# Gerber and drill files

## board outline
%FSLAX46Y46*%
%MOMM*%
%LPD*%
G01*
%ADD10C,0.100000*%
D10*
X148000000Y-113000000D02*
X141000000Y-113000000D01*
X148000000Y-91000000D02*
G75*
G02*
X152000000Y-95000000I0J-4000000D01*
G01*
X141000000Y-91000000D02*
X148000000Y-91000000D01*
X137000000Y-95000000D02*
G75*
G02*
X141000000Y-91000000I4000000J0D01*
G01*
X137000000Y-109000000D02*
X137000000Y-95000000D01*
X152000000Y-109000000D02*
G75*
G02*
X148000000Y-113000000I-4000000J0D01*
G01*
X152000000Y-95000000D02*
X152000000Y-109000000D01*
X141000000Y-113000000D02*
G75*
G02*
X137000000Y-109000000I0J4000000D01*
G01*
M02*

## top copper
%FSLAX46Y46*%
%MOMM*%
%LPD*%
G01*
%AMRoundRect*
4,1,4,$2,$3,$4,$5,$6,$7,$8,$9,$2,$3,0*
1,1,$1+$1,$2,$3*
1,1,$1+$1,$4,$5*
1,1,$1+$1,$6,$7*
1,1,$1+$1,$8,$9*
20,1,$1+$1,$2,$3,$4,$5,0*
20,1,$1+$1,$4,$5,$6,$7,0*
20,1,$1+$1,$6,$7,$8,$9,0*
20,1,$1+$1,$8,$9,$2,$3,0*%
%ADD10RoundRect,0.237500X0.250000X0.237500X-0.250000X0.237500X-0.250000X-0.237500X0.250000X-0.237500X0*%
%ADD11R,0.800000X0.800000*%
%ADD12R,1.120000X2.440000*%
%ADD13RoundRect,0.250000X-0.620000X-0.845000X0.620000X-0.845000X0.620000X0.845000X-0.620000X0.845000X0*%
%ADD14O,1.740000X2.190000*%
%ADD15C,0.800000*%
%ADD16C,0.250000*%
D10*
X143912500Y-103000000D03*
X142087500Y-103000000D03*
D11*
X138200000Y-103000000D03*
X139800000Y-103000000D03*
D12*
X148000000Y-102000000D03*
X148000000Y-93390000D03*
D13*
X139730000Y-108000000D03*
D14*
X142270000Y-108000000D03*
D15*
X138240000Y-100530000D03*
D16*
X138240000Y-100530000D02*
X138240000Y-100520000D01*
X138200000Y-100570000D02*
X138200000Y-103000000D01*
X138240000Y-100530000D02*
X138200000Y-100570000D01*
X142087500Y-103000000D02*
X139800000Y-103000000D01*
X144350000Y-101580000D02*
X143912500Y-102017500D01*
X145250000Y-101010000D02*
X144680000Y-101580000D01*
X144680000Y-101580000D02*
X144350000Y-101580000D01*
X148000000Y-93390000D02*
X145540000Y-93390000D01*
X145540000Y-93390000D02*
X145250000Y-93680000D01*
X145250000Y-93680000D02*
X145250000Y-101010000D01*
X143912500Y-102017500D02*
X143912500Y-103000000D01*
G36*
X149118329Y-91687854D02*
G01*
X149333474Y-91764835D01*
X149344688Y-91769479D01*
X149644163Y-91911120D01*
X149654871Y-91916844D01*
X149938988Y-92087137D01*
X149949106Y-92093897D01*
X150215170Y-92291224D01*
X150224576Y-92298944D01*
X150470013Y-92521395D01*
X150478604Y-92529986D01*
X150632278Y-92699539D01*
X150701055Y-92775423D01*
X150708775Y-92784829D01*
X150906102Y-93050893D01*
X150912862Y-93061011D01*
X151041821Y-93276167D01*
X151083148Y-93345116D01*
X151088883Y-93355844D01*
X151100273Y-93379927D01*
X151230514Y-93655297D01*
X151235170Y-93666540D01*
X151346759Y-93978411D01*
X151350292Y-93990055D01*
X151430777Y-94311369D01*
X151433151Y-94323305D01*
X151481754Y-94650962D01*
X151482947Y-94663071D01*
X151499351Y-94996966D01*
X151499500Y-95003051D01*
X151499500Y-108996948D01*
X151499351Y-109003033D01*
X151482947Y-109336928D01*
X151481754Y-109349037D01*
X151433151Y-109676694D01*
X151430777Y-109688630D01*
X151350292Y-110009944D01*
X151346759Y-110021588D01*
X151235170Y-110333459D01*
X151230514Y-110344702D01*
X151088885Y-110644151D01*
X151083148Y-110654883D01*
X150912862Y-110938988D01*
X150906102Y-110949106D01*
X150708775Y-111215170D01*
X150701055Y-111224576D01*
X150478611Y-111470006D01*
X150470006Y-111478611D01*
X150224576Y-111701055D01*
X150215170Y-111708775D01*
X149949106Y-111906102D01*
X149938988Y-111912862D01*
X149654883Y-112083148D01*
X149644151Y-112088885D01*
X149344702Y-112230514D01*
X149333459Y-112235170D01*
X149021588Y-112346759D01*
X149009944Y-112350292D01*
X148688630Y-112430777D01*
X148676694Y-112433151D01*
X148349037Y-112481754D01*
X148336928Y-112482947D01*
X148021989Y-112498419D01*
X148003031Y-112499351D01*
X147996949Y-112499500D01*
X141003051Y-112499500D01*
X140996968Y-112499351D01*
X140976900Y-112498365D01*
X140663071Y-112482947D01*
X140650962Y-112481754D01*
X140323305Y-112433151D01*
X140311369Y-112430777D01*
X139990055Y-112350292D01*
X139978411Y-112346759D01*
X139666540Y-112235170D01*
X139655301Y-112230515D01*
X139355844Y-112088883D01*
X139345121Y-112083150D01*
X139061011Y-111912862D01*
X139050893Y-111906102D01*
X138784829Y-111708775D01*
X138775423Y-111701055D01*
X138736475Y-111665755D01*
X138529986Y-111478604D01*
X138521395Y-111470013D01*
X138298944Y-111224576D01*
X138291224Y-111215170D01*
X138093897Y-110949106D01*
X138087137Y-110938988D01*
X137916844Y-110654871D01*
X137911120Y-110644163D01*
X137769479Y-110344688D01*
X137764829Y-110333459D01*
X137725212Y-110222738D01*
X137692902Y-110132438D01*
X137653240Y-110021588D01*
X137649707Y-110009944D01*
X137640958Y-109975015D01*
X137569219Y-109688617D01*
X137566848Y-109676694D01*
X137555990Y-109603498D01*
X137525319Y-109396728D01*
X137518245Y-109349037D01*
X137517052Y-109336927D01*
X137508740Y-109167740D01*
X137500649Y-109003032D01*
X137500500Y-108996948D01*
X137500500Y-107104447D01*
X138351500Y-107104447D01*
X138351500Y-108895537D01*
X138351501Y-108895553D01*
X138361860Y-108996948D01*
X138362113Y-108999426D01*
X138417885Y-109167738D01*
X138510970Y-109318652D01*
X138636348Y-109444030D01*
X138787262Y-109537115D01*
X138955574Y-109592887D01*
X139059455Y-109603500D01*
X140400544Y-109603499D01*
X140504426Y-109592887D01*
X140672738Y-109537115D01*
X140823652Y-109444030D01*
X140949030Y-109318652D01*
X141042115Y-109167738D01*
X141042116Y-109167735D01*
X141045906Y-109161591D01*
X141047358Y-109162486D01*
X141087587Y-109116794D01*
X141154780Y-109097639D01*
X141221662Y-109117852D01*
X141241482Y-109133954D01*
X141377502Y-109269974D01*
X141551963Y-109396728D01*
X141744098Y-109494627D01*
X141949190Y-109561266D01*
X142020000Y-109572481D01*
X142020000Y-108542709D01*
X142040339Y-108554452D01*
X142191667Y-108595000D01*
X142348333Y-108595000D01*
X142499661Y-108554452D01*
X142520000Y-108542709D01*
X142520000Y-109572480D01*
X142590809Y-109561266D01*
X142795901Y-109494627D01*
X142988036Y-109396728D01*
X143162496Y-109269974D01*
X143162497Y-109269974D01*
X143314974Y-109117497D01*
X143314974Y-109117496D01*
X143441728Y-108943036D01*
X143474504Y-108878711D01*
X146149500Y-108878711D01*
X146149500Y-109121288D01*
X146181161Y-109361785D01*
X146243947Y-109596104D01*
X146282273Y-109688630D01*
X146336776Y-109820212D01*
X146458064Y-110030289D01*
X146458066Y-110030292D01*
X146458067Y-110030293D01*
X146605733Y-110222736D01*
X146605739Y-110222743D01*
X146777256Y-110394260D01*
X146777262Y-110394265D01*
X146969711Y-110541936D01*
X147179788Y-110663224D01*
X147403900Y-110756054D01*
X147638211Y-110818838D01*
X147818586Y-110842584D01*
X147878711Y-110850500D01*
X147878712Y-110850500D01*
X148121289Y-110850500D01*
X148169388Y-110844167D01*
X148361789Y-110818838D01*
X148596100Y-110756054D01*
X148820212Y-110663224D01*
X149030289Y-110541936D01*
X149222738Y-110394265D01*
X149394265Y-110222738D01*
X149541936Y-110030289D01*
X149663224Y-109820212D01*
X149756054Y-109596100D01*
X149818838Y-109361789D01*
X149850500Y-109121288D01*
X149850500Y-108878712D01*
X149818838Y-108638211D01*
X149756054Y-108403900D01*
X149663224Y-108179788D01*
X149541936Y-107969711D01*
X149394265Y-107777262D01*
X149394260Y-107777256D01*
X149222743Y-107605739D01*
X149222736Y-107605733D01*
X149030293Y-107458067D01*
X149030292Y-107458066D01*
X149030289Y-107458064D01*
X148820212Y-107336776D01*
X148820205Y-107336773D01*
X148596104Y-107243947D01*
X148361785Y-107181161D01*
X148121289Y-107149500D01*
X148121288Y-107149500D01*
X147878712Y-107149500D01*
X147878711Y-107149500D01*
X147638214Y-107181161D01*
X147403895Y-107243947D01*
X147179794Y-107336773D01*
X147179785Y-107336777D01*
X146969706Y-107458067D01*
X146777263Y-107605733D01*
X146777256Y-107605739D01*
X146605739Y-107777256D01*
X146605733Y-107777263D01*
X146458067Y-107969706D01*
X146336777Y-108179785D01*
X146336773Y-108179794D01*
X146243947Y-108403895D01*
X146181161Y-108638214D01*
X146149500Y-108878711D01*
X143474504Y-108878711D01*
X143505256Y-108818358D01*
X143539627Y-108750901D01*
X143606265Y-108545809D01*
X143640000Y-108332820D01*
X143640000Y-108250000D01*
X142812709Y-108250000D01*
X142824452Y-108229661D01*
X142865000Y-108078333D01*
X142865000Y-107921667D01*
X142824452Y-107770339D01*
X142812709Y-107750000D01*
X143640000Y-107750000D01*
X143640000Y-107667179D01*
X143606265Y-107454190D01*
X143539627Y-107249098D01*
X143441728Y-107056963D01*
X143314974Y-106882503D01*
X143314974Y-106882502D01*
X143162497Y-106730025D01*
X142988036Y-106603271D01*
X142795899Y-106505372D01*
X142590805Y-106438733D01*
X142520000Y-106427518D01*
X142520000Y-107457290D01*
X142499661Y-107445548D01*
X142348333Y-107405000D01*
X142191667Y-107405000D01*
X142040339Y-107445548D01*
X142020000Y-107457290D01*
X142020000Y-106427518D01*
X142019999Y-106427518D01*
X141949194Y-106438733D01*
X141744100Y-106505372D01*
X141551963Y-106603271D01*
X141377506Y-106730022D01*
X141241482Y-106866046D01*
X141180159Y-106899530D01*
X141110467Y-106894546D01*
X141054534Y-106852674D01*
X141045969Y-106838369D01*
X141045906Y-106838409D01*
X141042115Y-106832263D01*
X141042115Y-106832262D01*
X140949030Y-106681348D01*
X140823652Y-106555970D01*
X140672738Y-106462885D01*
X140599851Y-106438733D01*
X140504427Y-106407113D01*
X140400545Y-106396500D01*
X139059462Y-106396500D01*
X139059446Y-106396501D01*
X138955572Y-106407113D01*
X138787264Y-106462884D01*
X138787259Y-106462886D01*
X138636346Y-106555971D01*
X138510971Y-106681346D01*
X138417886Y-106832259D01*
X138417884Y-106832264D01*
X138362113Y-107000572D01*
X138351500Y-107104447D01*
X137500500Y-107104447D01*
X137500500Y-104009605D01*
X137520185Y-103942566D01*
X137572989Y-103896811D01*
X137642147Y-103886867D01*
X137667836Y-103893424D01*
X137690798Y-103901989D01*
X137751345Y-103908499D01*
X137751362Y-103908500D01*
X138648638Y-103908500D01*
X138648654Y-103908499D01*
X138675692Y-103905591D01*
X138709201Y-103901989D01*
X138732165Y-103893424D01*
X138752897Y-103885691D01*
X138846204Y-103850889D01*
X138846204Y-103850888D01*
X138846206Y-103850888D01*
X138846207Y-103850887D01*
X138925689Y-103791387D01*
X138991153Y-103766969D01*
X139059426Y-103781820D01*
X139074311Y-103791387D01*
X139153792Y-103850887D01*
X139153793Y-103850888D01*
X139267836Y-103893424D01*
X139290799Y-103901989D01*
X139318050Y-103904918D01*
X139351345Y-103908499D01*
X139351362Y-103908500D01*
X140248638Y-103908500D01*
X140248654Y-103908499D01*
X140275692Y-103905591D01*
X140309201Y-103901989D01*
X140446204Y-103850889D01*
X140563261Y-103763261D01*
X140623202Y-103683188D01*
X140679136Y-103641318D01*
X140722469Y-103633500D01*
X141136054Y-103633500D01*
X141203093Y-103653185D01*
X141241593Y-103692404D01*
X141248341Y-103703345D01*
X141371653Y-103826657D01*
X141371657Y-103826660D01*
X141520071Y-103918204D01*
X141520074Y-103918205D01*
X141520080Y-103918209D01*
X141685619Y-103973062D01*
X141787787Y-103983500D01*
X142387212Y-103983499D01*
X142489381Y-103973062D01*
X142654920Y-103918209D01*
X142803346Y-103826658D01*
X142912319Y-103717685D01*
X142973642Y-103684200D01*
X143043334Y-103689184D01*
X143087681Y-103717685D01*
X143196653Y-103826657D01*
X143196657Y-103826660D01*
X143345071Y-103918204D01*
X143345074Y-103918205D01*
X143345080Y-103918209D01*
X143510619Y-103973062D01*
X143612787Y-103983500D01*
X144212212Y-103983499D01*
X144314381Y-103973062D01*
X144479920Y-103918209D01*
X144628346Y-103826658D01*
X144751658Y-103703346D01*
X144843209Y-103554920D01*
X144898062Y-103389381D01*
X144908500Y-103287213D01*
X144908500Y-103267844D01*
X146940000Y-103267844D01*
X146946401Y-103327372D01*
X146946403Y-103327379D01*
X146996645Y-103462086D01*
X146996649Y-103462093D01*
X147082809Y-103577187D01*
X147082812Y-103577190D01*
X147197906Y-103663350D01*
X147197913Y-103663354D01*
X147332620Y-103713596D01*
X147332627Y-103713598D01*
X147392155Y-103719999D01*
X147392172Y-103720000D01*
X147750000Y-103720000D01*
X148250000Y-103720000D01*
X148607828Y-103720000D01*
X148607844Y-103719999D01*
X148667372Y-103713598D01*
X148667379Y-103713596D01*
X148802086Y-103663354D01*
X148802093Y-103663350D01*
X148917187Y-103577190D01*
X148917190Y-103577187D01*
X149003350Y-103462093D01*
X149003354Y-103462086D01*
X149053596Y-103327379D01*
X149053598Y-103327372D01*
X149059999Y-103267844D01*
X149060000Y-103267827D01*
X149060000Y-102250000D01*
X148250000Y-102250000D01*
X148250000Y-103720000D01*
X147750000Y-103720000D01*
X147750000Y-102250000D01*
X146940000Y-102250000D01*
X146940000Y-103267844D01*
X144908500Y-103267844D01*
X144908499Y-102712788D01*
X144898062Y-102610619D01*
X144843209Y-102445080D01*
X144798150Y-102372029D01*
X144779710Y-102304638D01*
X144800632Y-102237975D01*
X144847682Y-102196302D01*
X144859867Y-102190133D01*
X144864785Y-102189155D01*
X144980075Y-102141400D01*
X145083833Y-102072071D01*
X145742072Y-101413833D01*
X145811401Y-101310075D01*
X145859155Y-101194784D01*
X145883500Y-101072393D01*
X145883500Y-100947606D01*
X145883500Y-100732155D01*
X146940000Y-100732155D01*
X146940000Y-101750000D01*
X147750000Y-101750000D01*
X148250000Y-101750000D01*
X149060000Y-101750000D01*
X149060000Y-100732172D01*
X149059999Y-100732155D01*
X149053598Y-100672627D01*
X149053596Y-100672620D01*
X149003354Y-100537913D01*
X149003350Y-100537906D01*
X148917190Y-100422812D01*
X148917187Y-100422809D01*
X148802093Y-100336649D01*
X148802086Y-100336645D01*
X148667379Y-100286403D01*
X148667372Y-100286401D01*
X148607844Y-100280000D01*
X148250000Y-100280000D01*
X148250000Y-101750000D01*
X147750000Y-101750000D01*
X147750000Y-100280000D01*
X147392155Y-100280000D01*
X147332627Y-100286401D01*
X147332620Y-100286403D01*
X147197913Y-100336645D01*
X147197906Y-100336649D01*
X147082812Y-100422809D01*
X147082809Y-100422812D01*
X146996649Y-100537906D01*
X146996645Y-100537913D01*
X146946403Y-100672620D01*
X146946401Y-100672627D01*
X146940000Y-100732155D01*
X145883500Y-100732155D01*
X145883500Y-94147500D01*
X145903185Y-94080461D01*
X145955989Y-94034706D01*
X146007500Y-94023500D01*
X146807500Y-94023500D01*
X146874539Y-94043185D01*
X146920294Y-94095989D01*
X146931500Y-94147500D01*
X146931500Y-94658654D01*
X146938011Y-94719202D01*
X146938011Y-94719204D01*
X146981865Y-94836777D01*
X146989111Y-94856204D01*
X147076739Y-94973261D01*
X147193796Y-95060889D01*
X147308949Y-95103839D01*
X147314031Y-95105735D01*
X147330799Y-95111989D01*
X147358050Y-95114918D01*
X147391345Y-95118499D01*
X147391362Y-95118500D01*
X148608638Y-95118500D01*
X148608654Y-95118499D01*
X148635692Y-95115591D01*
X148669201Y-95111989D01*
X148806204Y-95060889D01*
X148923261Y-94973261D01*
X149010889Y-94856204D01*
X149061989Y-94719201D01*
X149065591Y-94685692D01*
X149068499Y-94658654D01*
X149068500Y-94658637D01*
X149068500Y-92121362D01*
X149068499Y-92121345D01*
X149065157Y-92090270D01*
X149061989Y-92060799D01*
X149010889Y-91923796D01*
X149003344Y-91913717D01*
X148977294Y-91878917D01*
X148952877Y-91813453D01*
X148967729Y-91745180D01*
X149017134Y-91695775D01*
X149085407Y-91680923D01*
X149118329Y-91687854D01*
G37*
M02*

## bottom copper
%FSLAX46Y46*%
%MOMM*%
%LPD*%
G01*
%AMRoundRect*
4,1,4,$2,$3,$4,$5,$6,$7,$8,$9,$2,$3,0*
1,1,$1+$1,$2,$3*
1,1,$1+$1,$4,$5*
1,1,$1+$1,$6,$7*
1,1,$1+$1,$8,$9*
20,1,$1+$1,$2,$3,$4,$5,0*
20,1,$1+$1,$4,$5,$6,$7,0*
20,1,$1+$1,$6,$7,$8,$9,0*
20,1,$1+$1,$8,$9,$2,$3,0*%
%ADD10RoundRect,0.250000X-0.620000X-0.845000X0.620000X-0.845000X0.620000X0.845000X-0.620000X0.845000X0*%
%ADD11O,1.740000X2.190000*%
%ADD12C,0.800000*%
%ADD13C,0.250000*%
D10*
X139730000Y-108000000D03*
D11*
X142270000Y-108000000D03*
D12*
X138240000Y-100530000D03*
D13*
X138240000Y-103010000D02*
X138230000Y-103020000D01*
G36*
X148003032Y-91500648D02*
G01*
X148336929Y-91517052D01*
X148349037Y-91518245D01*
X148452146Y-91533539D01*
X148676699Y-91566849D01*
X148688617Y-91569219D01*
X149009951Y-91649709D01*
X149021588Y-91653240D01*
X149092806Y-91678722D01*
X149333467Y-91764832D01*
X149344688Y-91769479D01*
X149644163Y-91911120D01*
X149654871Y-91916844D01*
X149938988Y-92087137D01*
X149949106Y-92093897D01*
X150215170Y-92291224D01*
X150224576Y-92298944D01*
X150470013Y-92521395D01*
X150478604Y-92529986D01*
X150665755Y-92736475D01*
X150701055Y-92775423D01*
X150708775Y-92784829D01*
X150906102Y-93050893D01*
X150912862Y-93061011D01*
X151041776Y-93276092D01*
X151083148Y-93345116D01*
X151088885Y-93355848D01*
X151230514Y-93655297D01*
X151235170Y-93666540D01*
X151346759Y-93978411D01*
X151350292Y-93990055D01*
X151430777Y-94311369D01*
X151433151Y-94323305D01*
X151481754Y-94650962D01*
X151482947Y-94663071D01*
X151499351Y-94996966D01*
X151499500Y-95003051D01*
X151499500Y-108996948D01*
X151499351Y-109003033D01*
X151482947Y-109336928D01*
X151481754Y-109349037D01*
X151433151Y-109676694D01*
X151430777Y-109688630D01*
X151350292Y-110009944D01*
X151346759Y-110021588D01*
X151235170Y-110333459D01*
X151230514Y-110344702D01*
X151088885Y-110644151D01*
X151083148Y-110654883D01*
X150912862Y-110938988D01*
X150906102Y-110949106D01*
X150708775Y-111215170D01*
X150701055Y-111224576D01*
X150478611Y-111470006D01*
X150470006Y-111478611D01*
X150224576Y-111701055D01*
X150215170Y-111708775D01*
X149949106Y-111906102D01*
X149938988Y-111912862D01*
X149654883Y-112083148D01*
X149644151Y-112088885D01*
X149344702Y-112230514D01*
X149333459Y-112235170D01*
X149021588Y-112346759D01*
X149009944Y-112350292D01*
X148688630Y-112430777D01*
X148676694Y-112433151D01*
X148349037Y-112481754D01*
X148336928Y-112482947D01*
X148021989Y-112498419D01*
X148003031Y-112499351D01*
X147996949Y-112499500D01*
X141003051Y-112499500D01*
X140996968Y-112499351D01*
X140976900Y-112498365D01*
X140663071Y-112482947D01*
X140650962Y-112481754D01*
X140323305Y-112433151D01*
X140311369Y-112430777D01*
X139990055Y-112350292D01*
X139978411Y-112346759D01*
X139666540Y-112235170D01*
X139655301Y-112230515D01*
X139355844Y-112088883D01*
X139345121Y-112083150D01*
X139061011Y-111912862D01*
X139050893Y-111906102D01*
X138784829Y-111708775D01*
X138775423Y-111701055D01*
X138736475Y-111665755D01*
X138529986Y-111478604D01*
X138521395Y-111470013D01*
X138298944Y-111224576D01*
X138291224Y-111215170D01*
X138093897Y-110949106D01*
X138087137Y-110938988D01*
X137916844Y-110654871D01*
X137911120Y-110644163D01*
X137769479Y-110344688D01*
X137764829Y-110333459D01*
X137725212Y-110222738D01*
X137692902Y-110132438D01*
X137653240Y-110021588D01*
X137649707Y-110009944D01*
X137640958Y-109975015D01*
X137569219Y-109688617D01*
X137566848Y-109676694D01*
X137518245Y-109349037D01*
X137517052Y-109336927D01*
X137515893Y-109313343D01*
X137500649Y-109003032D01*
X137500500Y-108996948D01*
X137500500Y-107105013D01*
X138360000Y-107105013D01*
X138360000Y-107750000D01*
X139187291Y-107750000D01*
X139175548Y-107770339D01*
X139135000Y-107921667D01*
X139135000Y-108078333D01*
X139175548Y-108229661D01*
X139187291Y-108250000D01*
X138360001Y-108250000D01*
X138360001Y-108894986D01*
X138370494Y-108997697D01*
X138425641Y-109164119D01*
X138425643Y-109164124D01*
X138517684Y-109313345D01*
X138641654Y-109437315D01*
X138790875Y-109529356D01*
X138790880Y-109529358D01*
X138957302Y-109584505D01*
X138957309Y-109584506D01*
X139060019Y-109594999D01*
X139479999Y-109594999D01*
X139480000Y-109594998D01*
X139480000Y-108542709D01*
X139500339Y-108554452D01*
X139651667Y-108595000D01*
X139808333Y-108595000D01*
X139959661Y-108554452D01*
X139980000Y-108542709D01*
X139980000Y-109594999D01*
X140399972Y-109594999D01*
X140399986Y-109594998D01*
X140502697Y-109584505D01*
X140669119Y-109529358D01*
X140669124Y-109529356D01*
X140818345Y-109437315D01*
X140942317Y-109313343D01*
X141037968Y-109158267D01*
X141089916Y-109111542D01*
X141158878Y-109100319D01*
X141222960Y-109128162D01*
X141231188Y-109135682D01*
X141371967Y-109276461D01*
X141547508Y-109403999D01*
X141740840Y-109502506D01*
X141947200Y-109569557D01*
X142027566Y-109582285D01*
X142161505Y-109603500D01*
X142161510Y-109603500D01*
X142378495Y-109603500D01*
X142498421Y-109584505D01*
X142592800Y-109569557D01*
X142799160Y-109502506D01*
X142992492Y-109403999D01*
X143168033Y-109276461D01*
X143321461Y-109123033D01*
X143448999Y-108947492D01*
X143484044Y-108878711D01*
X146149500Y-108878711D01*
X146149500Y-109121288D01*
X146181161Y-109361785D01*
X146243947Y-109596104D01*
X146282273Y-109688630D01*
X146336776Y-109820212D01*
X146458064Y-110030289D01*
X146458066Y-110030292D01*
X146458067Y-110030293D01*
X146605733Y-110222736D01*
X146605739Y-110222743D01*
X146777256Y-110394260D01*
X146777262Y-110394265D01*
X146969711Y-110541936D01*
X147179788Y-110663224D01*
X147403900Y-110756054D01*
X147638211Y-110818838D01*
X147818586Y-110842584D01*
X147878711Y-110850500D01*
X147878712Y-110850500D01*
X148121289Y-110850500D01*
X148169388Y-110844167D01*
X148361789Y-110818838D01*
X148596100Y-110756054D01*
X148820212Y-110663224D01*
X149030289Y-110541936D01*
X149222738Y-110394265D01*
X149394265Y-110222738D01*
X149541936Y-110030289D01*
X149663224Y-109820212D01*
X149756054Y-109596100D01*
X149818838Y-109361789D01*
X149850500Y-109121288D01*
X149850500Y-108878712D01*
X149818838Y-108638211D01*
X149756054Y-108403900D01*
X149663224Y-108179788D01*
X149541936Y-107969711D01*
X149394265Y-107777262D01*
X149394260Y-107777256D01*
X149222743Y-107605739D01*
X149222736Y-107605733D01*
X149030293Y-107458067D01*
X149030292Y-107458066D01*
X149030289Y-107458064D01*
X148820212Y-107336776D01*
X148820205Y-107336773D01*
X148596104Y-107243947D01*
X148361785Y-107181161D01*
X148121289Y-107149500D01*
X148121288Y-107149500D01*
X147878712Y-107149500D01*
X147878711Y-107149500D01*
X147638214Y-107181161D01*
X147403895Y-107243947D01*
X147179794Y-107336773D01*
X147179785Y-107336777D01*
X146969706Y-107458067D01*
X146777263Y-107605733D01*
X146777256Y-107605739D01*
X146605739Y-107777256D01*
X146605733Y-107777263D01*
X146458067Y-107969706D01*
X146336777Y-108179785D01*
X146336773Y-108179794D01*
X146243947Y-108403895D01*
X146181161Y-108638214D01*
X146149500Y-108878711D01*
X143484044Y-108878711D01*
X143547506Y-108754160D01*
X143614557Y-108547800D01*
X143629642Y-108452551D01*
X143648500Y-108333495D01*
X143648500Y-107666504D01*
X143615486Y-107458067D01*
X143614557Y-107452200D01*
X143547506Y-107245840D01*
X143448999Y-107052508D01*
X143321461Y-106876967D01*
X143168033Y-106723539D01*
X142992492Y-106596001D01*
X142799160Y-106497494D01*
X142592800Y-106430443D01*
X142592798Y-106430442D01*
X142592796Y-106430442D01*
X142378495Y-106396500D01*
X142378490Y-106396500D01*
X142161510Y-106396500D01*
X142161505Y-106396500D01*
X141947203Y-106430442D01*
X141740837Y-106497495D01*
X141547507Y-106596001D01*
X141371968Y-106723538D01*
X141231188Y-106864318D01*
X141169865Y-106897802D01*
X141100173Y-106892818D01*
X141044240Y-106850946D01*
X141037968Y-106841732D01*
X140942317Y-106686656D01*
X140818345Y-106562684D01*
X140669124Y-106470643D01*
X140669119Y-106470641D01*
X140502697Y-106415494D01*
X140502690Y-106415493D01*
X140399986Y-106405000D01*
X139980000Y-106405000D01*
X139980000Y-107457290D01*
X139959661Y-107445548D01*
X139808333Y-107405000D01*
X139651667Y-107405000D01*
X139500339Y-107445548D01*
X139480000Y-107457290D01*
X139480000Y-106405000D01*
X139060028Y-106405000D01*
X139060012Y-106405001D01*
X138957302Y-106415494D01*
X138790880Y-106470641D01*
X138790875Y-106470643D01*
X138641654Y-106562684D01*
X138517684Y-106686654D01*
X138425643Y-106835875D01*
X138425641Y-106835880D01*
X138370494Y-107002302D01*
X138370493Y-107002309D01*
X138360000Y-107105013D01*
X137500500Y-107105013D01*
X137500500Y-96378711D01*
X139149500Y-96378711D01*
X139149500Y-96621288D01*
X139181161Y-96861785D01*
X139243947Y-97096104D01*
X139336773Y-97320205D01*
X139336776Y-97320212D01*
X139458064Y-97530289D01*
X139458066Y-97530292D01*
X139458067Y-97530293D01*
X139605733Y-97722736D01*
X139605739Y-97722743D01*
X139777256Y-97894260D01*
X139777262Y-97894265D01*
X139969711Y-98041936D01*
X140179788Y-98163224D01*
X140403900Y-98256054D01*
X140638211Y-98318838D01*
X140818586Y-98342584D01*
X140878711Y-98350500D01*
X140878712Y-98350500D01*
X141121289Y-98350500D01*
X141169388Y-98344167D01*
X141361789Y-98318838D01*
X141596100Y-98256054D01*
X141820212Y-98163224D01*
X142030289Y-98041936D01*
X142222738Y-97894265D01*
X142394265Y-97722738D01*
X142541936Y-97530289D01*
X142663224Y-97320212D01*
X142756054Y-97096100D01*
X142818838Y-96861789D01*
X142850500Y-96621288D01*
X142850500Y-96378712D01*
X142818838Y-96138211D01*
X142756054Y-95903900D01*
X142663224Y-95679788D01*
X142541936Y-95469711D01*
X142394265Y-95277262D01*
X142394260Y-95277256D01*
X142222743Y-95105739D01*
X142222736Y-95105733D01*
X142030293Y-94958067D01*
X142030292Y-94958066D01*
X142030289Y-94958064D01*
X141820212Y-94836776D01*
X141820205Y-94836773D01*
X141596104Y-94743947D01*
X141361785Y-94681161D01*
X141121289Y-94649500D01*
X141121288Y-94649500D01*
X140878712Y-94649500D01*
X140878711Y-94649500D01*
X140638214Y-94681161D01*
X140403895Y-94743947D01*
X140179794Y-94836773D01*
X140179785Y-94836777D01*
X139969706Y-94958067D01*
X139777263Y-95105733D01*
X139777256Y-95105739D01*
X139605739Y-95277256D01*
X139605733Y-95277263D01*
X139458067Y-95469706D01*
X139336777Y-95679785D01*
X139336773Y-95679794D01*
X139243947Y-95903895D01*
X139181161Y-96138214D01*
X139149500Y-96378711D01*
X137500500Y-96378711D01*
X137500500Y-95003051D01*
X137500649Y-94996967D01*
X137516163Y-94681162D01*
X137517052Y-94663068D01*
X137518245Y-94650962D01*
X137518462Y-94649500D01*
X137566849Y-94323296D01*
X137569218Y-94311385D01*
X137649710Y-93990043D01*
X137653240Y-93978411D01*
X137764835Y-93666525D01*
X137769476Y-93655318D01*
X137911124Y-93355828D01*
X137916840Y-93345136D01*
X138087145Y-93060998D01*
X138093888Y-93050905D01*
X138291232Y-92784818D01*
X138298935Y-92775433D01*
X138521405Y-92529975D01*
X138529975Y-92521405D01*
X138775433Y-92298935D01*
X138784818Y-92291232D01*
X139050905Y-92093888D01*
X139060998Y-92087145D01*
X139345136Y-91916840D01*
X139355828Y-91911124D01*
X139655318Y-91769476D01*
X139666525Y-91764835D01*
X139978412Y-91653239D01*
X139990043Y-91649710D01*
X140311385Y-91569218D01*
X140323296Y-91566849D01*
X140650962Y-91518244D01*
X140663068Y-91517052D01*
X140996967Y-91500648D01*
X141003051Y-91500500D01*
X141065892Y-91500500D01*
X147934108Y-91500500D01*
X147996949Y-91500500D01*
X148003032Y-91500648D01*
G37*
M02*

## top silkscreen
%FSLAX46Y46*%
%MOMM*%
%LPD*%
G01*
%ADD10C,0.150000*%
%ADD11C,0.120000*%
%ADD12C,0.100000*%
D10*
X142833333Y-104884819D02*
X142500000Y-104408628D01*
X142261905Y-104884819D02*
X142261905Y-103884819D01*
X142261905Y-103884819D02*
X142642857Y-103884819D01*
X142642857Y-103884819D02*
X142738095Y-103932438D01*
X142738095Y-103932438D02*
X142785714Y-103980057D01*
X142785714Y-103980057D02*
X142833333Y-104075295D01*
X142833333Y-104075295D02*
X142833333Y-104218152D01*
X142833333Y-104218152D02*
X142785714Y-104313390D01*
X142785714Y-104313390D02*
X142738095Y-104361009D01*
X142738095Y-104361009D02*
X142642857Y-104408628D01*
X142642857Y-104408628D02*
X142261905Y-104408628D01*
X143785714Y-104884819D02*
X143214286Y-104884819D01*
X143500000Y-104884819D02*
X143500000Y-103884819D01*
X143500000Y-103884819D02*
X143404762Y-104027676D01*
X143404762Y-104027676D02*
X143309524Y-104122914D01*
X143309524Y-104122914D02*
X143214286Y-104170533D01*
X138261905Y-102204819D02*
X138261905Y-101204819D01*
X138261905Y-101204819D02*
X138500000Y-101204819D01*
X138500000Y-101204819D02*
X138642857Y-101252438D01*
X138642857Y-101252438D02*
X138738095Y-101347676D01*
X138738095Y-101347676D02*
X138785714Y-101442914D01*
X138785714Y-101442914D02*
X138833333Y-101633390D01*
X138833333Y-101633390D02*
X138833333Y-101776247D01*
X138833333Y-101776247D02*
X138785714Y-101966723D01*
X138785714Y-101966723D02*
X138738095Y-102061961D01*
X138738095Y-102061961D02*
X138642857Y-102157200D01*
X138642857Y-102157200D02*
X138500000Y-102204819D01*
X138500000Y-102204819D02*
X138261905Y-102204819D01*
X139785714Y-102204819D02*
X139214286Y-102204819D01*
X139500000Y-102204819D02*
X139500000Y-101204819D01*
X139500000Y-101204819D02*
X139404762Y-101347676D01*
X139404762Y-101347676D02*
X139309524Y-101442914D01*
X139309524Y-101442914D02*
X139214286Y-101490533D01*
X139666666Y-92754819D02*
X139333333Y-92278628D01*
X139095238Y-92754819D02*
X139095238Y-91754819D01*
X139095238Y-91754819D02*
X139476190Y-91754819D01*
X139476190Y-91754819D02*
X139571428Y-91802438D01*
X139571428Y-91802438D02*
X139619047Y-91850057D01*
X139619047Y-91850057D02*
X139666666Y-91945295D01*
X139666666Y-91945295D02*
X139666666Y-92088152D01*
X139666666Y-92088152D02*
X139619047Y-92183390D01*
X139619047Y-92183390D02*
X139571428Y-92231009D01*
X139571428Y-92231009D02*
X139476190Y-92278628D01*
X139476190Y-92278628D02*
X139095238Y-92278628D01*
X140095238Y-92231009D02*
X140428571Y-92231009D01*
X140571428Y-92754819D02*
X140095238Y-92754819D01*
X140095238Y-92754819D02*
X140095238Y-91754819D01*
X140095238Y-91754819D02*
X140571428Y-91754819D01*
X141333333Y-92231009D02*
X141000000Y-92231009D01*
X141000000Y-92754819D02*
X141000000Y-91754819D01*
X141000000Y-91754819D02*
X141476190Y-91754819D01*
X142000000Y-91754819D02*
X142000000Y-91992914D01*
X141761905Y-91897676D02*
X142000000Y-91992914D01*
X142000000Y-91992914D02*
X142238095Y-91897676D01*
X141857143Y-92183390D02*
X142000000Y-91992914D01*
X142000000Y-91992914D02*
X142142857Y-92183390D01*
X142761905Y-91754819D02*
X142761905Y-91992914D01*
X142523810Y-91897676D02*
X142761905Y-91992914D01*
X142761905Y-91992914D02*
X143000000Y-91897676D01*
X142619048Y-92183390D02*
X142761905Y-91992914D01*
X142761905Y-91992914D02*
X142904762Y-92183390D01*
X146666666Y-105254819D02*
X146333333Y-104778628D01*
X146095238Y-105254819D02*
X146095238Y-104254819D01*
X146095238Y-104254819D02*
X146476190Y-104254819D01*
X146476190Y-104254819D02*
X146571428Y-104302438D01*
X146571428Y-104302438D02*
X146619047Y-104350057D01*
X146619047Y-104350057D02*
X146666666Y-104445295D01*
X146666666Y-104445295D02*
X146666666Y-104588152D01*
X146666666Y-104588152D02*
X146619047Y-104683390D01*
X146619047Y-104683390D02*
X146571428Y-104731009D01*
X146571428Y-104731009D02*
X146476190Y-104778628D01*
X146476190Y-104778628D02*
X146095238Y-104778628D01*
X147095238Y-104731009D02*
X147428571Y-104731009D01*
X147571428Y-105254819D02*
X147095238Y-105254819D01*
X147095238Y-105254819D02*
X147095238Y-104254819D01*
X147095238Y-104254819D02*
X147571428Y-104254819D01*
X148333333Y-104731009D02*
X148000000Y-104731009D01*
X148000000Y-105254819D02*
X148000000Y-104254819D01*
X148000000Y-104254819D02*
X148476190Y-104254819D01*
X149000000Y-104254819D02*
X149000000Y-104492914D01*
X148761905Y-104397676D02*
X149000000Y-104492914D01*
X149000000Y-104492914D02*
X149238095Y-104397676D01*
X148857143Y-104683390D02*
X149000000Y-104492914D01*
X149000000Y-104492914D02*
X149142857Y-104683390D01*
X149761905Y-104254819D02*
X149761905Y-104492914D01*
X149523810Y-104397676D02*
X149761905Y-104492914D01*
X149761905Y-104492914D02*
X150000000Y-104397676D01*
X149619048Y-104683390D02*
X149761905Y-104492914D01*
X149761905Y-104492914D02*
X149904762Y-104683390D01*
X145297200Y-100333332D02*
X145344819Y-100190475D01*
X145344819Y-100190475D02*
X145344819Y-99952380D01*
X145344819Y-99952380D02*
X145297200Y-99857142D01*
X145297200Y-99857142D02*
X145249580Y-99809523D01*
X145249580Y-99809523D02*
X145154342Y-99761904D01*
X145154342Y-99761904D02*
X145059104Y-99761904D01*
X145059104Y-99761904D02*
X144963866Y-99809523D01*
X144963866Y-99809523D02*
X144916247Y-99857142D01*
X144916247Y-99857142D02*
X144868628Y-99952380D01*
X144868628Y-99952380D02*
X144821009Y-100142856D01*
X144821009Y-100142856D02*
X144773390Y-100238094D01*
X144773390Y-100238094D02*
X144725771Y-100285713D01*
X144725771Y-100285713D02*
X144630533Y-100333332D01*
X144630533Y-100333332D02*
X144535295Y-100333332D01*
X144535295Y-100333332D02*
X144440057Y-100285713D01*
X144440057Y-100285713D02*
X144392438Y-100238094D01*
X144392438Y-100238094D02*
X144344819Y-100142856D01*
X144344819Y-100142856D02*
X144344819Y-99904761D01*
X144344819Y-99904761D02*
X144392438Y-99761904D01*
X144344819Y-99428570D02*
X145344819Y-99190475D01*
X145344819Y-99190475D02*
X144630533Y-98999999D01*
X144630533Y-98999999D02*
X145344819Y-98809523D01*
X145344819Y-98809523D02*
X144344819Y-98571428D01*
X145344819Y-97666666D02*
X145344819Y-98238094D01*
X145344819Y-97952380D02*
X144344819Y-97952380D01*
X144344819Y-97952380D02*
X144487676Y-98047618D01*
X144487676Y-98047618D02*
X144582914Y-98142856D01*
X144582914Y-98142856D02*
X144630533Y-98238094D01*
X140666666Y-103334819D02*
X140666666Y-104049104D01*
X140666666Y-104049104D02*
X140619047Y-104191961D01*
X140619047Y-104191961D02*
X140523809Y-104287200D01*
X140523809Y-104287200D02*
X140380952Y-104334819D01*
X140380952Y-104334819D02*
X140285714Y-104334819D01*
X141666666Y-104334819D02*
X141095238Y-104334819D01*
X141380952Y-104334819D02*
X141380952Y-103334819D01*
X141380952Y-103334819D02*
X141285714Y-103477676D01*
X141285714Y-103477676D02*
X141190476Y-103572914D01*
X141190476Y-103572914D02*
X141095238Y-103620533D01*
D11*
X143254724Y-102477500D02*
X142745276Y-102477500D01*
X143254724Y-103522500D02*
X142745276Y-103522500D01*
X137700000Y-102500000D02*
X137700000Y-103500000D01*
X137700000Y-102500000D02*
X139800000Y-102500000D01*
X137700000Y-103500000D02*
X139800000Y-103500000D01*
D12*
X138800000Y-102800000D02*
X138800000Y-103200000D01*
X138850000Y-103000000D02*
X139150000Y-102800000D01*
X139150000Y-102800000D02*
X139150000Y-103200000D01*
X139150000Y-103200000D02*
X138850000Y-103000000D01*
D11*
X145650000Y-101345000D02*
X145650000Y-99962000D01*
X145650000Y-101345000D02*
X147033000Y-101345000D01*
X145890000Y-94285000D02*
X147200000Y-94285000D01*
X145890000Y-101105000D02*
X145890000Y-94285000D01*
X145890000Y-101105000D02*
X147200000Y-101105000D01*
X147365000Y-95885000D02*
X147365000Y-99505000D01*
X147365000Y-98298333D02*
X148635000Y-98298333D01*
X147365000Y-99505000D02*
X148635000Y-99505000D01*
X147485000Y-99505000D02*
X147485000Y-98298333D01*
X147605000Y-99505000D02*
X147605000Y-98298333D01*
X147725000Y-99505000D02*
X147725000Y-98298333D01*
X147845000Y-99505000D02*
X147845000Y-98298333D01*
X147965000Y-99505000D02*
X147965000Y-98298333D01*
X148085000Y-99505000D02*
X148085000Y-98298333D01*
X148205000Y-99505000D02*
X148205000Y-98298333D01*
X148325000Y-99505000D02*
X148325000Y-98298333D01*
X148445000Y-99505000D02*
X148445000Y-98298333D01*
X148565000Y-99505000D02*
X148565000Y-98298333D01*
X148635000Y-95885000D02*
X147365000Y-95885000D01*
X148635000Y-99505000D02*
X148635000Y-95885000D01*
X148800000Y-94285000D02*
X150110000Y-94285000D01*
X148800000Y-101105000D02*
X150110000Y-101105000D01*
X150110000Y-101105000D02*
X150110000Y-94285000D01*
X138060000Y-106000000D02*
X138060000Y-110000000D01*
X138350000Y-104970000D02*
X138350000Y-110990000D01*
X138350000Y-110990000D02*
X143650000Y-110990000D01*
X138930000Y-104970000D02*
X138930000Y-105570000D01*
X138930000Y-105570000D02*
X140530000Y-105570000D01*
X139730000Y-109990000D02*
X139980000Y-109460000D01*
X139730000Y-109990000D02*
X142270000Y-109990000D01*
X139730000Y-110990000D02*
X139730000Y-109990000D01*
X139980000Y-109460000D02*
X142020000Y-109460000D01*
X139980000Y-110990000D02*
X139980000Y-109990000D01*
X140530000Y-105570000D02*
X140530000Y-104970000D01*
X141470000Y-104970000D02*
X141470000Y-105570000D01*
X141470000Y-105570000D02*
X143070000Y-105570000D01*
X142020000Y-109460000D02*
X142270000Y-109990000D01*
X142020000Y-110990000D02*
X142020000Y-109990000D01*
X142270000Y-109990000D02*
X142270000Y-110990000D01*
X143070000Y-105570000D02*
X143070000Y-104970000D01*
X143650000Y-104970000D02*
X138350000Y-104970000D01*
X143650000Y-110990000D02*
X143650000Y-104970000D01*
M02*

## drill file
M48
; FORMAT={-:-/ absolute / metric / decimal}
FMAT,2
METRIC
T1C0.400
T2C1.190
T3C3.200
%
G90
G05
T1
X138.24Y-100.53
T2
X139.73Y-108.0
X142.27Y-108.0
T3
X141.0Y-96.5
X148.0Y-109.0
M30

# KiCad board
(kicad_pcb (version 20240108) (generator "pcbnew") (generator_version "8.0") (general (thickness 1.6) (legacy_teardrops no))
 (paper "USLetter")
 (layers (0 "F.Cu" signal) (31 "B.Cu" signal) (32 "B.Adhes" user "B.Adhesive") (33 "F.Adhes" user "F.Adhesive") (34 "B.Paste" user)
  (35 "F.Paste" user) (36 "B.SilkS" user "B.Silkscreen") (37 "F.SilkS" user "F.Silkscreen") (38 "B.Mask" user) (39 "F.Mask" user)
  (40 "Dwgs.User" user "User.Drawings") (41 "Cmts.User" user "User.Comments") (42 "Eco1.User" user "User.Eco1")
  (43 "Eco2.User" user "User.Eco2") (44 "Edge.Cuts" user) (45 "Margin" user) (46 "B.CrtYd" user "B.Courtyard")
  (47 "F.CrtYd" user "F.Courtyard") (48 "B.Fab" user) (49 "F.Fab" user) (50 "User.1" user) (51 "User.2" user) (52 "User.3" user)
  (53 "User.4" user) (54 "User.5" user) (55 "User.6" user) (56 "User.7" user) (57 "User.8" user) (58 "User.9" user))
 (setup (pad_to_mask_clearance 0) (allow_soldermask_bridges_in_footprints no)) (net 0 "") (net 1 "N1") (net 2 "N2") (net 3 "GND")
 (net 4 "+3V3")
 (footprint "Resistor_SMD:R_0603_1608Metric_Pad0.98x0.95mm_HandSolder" (layer "F.Cu") (at 143 103 180)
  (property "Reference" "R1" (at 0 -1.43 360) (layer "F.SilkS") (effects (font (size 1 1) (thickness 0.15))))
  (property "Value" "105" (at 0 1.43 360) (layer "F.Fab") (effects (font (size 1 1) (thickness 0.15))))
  (fp_line (start -0.254724 0.5225) (end 0.254724 0.5225) (stroke (width 0.12) (type solid)) (layer "F.SilkS"))
  (fp_line (start -0.254724 -0.5225) (end 0.254724 -0.5225) (stroke (width 0.12) (type solid)) (layer "F.SilkS"))
  (pad "1" smd roundrect (at -0.9125 0 180) (size 0.975 0.95) (layers "F.Cu" "F.Paste" "F.Mask") (roundrect_rratio 0.25) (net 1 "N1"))
  (pad "2" smd roundrect (at 0.9125 0 180) (size 0.975 0.95) (layers "F.Cu" "F.Paste" "F.Mask") (roundrect_rratio 0.25) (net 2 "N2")))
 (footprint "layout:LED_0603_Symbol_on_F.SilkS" (layer "F.Cu") (at 139 103)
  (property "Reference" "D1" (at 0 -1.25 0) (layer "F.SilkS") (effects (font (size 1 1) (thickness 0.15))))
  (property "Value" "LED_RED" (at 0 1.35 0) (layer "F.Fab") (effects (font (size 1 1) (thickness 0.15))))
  (fp_line (start -1.3 -0.5) (end -1.3 0.5) (stroke (width 0.12) (type solid)) (layer "F.SilkS"))
  (fp_line (start -1.3 -0.5) (end 0.8 -0.5) (stroke (width 0.12) (type solid)) (layer "F.SilkS"))
  (fp_line (start -1.3 0.5) (end 0.8 0.5) (stroke (width 0.12) (type solid)) (layer "F.SilkS"))
  (fp_line (start -0.2 -0.2) (end -0.2 0.2) (stroke (width 0.1) (type solid)) (layer "F.SilkS"))
  (fp_line (start -0.15 0) (end 0.15 -0.2) (stroke (width 0.1) (type solid)) (layer "F.SilkS"))
  (fp_line (start 0.15 -0.2) (end 0.15 0.2) (stroke (width 0.1) (type solid)) (layer "F.SilkS"))
  (fp_line (start 0.15 0.2) (end -0.15 0) (stroke (width 0.1) (type solid)) (layer "F.SilkS"))
  (pad "1" smd rect (at -0.8 0 180) (size 0.8 0.8) (layers "F.Cu" "F.Paste" "F.Mask") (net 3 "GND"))
  (pad "2" smd rect (at 0.8 0 180) (size 0.8 0.8) (layers "F.Cu" "F.Paste" "F.Mask") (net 2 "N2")))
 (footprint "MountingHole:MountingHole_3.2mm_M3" (layer "F.Cu") (at 141 96.5)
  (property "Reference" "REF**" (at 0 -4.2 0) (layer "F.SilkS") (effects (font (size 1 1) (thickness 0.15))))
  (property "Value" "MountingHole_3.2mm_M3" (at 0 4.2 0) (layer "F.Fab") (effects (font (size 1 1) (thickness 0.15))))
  (pad "" np_thru_hole circle (at 0 0) (size 3.2 3.2) (drill 3.2) (layers "*.Cu" "*.Mask")))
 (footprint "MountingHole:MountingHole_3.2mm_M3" (layer "F.Cu") (at 148 109)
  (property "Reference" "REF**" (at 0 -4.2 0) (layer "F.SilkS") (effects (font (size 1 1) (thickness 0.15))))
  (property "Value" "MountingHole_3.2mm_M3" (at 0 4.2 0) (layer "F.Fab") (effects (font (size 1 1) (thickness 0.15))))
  (pad "" np_thru_hole circle (at 0 0) (size 3.2 3.2) (drill 3.2) (layers "*.Cu" "*.Mask")))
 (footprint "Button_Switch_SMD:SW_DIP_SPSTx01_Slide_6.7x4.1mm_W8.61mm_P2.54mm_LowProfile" (layer "F.Cu") (at 148 97.695 90)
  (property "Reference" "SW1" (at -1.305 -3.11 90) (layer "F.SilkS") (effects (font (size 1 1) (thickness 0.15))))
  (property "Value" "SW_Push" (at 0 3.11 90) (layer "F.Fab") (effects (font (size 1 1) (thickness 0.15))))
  (fp_line (start -3.65 -2.35) (end -2.267 -2.35) (stroke (width 0.12) (type solid)) (layer "F.SilkS"))
  (fp_line (start -3.65 -2.35) (end -3.65 -0.967) (stroke (width 0.12) (type solid)) (layer "F.SilkS"))
  (fp_line (start 3.41 -2.11) (end 3.41 -0.8) (stroke (width 0.12) (type solid)) (layer "F.SilkS"))
  (fp_line (start -3.41 -2.11) (end 3.41 -2.11) (stroke (width 0.12) (type solid)) (layer "F.SilkS"))
  (fp_line (start -3.41 -2.11) (end -3.41 -0.8) (stroke (width 0.12) (type solid)) (layer "F.SilkS"))
  (fp_line (start 1.81 -0.635) (end -1.81 -0.635) (stroke (width 0.12) (type solid)) (layer "F.SilkS"))
  (fp_line (start -0.603333 -0.635) (end -0.603333 0.635) (stroke (width 0.12) (type solid)) (layer "F.SilkS"))
  (fp_line (start -1.81 -0.635) (end -1.81 0.635) (stroke (width 0.12) (type solid)) (layer "F.SilkS"))
  (fp_line (start -1.81 -0.515) (end -0.603333 -0.515) (stroke (width 0.12) (type solid)) (layer "F.SilkS"))
  (fp_line (start -1.81 -0.395) (end -0.603333 -0.395) (stroke (width 0.12) (type solid)) (layer "F.SilkS"))
  (fp_line (start -1.81 -0.275) (end -0.603333 -0.275) (stroke (width 0.12) (type solid)) (layer "F.SilkS"))
  (fp_line (start -1.81 -0.155) (end -0.603333 -0.155) (stroke (width 0.12) (type solid)) (layer "F.SilkS"))
  (fp_line (start -1.81 -0.035) (end -0.603333 -0.035) (stroke (width 0.12) (type solid)) (layer "F.SilkS"))
  (fp_line (start -1.81 0.085) (end -0.603333 0.085) (stroke (width 0.12) (type solid)) (layer "F.SilkS"))
  (fp_line (start -1.81 0.205) (end -0.603333 0.205) (stroke (width 0.12) (type solid)) (layer "F.SilkS"))
  (fp_line (start -1.81 0.325) (end -0.603333 0.325) (stroke (width 0.12) (type solid)) (layer "F.SilkS"))
  (fp_line (start -1.81 0.445) (end -0.603333 0.445) (stroke (width 0.12) (type solid)) (layer "F.SilkS"))
  (fp_line (start -1.81 0.565) (end -0.603333 0.565) (stroke (width 0.12) (type solid)) (layer "F.SilkS"))
  (fp_line (start 1.81 0.635) (end 1.81 -0.635) (stroke (width 0.12) (type solid)) (layer "F.SilkS"))
  (fp_line (start -1.81 0.635) (end 1.81 0.635) (stroke (width 0.12) (type solid)) (layer "F.SilkS"))
  (fp_line (start 3.41 0.8) (end 3.41 2.11) (stroke (width 0.12) (type solid)) (layer "F.SilkS"))
  (fp_line (start -3.41 0.8) (end -3.41 2.11) (stroke (width 0.12) (type solid)) (layer "F.SilkS"))
  (fp_line (start -3.41 2.11) (end 3.41 2.11) (stroke (width 0.12) (type solid)) (layer "F.SilkS"))
  (pad "1" smd rect (at -4.305 0 90) (size 2.44 1.12) (layers "F.Cu" "F.Paste" "F.Mask") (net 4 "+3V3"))
  (pad "2" smd rect (at 4.305 0 90) (size 2.44 1.12) (layers "F.Cu" "F.Paste" "F.Mask") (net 1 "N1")))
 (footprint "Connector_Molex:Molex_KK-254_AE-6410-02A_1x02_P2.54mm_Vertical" (layer "F.Cu") (at 139.73 108)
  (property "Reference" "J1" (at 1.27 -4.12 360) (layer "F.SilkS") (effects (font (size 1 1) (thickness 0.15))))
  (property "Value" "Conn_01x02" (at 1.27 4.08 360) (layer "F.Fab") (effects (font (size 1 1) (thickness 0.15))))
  (fp_line (start -1.67 -2) (end -1.67 2) (stroke (width 0.12) (type solid)) (layer "F.SilkS"))
  (fp_line (start -1.38 -3.03) (end -1.38 2.99) (stroke (width 0.12) (type solid)) (layer "F.SilkS"))
  (fp_line (start -1.38 2.99) (end 3.92 2.99) (stroke (width 0.12) (type solid)) (layer "F.SilkS"))
  (fp_line (start -0.8 -3.03) (end -0.8 -2.43) (stroke (width 0.12) (type solid)) (layer "F.SilkS"))
  (fp_line (start -0.8 -2.43) (end 0.8 -2.43) (stroke (width 0.12) (type solid)) (layer "F.SilkS"))
  (fp_line (start 0 1.99) (end 0.25 1.46) (stroke (width 0.12) (type solid)) (layer "F.SilkS"))
  (fp_line (start 0 1.99) (end 2.54 1.99) (stroke (width 0.12) (type solid)) (layer "F.SilkS"))
  (fp_line (start 0 2.99) (end 0 1.99) (stroke (width 0.12) (type solid)) (layer "F.SilkS"))
  (fp_line (start 0.25 1.46) (end 2.29 1.46) (stroke (width 0.12) (type solid)) (layer "F.SilkS"))
  (fp_line (start 0.25 2.99) (end 0.25 1.99) (stroke (width 0.12) (type solid)) (layer "F.SilkS"))
  (fp_line (start 0.8 -2.43) (end 0.8 -3.03) (stroke (width 0.12) (type solid)) (layer "F.SilkS"))
  (fp_line (start 1.74 -3.03) (end 1.74 -2.43) (stroke (width 0.12) (type solid)) (layer "F.SilkS"))
  (fp_line (start 1.74 -2.43) (end 3.34 -2.43) (stroke (width 0.12) (type solid)) (layer "F.SilkS"))
  (fp_line (start 2.29 1.46) (end 2.54 1.99) (stroke (width 0.12) (type solid)) (layer "F.SilkS"))
  (fp_line (start 2.29 2.99) (end 2.29 1.99) (stroke (width 0.12) (type solid)) (layer "F.SilkS"))
  (fp_line (start 2.54 1.99) (end 2.54 2.99) (stroke (width 0.12) (type solid)) (layer "F.SilkS"))
  (fp_line (start 3.34 -2.43) (end 3.34 -3.03) (stroke (width 0.12) (type solid)) (layer "F.SilkS"))
  (fp_line (start 3.92 -3.03) (end -1.38 -3.03) (stroke (width 0.12) (type solid)) (layer "F.SilkS"))
  (fp_line (start 3.92 2.99) (end 3.92 -3.03) (stroke (width 0.12) (type solid)) (layer "F.SilkS"))
  (pad "1" thru_hole roundrect (at 0 0) (size 1.74 2.19) (drill 1.19) (layers "*.Cu" "*.Mask") (remove_unused_layers no)
   (roundrect_rratio 0.143678) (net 3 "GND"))
  (pad "2" thru_hole oval (at 2.54 0) (size 1.74 2.19) (drill 1.19) (layers "*.Cu" "*.Mask") (remove_unused_layers no) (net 4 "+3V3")))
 (gr_line (start 148 113) (end 141 113) (stroke (width 0.1) (type default)) (layer "Edge.Cuts"))
 (gr_arc (start 148 91) (mid 150.828427 92.171573) (end 152 95) (stroke (width 0.1) (type default)) (layer "Edge.Cuts"))
 (gr_line (start 141 91) (end 148 91) (stroke (width 0.1) (type default)) (layer "Edge.Cuts"))
 (gr_arc (start 137 95) (mid 138.171573 92.171573) (end 141 91) (stroke (width 0.1) (type default)) (layer "Edge.Cuts"))
 (gr_line (start 137 109) (end 137 95) (stroke (width 0.1) (type default)) (layer "Edge.Cuts"))
 (gr_arc (start 152 109) (mid 150.828427 111.828427) (end 148 113) (stroke (width 0.1) (type default)) (layer "Edge.Cuts"))
 (gr_line (start 152 95) (end 152 109) (stroke (width 0.1) (type default)) (layer "Edge.Cuts"))
 (gr_arc (start 141 113) (mid 138.171573 111.828427) (end 137 109) (stroke (width 0.1) (type default)) (layer "Edge.Cuts"))
 (segment (start 138.24 100.53) (end 138.24 100.52) (width 0.25) (layer "F.Cu") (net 3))
 (segment (start 138.2 100.57) (end 138.2 103) (width 0.25) (layer "F.Cu") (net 3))
 (segment (start 138.24 100.53) (end 138.2 100.57) (width 0.25) (layer "F.Cu") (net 3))
 (via (at 138.24 100.53) (size 0.8) (drill 0.4) (layers "F.Cu" "B.Cu") (free yes) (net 3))
 (segment (start 138.24 103.01) (end 138.23 103.02) (width 0.25) (layer "B.Cu") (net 3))
 (segment (start 142.0875 103) (end 139.8 103) (width 0.25) (layer "F.Cu") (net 2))
 (segment (start 144.35 101.58) (end 143.9125 102.0175) (width 0.25) (layer "F.Cu") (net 1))
 (segment (start 145.25 101.01) (end 144.68 101.58) (width 0.25) (layer "F.Cu") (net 1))
 (segment (start 144.68 101.58) (end 144.35 101.58) (width 0.25) (layer "F.Cu") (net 1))
 (segment (start 148 93.39) (end 145.54 93.39) (width 0.25) (layer "F.Cu") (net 1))
 (segment (start 145.54 93.39) (end 145.25 93.68) (width 0.25) (layer "F.Cu") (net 1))
 (segment (start 145.25 93.68) (end 145.25 101.01) (width 0.25) (layer "F.Cu") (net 1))
 (segment (start 143.9125 102.0175) (end 143.9125 103) (width 0.25) (layer "F.Cu") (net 1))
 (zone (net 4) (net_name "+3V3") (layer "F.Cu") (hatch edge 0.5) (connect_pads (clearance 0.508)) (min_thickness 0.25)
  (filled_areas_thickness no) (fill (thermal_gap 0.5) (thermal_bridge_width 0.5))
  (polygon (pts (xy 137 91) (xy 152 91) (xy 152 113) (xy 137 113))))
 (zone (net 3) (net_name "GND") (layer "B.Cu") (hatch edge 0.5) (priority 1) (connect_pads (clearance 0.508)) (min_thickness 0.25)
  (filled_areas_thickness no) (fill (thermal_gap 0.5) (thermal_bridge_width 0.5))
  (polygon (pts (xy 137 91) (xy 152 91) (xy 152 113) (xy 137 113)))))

